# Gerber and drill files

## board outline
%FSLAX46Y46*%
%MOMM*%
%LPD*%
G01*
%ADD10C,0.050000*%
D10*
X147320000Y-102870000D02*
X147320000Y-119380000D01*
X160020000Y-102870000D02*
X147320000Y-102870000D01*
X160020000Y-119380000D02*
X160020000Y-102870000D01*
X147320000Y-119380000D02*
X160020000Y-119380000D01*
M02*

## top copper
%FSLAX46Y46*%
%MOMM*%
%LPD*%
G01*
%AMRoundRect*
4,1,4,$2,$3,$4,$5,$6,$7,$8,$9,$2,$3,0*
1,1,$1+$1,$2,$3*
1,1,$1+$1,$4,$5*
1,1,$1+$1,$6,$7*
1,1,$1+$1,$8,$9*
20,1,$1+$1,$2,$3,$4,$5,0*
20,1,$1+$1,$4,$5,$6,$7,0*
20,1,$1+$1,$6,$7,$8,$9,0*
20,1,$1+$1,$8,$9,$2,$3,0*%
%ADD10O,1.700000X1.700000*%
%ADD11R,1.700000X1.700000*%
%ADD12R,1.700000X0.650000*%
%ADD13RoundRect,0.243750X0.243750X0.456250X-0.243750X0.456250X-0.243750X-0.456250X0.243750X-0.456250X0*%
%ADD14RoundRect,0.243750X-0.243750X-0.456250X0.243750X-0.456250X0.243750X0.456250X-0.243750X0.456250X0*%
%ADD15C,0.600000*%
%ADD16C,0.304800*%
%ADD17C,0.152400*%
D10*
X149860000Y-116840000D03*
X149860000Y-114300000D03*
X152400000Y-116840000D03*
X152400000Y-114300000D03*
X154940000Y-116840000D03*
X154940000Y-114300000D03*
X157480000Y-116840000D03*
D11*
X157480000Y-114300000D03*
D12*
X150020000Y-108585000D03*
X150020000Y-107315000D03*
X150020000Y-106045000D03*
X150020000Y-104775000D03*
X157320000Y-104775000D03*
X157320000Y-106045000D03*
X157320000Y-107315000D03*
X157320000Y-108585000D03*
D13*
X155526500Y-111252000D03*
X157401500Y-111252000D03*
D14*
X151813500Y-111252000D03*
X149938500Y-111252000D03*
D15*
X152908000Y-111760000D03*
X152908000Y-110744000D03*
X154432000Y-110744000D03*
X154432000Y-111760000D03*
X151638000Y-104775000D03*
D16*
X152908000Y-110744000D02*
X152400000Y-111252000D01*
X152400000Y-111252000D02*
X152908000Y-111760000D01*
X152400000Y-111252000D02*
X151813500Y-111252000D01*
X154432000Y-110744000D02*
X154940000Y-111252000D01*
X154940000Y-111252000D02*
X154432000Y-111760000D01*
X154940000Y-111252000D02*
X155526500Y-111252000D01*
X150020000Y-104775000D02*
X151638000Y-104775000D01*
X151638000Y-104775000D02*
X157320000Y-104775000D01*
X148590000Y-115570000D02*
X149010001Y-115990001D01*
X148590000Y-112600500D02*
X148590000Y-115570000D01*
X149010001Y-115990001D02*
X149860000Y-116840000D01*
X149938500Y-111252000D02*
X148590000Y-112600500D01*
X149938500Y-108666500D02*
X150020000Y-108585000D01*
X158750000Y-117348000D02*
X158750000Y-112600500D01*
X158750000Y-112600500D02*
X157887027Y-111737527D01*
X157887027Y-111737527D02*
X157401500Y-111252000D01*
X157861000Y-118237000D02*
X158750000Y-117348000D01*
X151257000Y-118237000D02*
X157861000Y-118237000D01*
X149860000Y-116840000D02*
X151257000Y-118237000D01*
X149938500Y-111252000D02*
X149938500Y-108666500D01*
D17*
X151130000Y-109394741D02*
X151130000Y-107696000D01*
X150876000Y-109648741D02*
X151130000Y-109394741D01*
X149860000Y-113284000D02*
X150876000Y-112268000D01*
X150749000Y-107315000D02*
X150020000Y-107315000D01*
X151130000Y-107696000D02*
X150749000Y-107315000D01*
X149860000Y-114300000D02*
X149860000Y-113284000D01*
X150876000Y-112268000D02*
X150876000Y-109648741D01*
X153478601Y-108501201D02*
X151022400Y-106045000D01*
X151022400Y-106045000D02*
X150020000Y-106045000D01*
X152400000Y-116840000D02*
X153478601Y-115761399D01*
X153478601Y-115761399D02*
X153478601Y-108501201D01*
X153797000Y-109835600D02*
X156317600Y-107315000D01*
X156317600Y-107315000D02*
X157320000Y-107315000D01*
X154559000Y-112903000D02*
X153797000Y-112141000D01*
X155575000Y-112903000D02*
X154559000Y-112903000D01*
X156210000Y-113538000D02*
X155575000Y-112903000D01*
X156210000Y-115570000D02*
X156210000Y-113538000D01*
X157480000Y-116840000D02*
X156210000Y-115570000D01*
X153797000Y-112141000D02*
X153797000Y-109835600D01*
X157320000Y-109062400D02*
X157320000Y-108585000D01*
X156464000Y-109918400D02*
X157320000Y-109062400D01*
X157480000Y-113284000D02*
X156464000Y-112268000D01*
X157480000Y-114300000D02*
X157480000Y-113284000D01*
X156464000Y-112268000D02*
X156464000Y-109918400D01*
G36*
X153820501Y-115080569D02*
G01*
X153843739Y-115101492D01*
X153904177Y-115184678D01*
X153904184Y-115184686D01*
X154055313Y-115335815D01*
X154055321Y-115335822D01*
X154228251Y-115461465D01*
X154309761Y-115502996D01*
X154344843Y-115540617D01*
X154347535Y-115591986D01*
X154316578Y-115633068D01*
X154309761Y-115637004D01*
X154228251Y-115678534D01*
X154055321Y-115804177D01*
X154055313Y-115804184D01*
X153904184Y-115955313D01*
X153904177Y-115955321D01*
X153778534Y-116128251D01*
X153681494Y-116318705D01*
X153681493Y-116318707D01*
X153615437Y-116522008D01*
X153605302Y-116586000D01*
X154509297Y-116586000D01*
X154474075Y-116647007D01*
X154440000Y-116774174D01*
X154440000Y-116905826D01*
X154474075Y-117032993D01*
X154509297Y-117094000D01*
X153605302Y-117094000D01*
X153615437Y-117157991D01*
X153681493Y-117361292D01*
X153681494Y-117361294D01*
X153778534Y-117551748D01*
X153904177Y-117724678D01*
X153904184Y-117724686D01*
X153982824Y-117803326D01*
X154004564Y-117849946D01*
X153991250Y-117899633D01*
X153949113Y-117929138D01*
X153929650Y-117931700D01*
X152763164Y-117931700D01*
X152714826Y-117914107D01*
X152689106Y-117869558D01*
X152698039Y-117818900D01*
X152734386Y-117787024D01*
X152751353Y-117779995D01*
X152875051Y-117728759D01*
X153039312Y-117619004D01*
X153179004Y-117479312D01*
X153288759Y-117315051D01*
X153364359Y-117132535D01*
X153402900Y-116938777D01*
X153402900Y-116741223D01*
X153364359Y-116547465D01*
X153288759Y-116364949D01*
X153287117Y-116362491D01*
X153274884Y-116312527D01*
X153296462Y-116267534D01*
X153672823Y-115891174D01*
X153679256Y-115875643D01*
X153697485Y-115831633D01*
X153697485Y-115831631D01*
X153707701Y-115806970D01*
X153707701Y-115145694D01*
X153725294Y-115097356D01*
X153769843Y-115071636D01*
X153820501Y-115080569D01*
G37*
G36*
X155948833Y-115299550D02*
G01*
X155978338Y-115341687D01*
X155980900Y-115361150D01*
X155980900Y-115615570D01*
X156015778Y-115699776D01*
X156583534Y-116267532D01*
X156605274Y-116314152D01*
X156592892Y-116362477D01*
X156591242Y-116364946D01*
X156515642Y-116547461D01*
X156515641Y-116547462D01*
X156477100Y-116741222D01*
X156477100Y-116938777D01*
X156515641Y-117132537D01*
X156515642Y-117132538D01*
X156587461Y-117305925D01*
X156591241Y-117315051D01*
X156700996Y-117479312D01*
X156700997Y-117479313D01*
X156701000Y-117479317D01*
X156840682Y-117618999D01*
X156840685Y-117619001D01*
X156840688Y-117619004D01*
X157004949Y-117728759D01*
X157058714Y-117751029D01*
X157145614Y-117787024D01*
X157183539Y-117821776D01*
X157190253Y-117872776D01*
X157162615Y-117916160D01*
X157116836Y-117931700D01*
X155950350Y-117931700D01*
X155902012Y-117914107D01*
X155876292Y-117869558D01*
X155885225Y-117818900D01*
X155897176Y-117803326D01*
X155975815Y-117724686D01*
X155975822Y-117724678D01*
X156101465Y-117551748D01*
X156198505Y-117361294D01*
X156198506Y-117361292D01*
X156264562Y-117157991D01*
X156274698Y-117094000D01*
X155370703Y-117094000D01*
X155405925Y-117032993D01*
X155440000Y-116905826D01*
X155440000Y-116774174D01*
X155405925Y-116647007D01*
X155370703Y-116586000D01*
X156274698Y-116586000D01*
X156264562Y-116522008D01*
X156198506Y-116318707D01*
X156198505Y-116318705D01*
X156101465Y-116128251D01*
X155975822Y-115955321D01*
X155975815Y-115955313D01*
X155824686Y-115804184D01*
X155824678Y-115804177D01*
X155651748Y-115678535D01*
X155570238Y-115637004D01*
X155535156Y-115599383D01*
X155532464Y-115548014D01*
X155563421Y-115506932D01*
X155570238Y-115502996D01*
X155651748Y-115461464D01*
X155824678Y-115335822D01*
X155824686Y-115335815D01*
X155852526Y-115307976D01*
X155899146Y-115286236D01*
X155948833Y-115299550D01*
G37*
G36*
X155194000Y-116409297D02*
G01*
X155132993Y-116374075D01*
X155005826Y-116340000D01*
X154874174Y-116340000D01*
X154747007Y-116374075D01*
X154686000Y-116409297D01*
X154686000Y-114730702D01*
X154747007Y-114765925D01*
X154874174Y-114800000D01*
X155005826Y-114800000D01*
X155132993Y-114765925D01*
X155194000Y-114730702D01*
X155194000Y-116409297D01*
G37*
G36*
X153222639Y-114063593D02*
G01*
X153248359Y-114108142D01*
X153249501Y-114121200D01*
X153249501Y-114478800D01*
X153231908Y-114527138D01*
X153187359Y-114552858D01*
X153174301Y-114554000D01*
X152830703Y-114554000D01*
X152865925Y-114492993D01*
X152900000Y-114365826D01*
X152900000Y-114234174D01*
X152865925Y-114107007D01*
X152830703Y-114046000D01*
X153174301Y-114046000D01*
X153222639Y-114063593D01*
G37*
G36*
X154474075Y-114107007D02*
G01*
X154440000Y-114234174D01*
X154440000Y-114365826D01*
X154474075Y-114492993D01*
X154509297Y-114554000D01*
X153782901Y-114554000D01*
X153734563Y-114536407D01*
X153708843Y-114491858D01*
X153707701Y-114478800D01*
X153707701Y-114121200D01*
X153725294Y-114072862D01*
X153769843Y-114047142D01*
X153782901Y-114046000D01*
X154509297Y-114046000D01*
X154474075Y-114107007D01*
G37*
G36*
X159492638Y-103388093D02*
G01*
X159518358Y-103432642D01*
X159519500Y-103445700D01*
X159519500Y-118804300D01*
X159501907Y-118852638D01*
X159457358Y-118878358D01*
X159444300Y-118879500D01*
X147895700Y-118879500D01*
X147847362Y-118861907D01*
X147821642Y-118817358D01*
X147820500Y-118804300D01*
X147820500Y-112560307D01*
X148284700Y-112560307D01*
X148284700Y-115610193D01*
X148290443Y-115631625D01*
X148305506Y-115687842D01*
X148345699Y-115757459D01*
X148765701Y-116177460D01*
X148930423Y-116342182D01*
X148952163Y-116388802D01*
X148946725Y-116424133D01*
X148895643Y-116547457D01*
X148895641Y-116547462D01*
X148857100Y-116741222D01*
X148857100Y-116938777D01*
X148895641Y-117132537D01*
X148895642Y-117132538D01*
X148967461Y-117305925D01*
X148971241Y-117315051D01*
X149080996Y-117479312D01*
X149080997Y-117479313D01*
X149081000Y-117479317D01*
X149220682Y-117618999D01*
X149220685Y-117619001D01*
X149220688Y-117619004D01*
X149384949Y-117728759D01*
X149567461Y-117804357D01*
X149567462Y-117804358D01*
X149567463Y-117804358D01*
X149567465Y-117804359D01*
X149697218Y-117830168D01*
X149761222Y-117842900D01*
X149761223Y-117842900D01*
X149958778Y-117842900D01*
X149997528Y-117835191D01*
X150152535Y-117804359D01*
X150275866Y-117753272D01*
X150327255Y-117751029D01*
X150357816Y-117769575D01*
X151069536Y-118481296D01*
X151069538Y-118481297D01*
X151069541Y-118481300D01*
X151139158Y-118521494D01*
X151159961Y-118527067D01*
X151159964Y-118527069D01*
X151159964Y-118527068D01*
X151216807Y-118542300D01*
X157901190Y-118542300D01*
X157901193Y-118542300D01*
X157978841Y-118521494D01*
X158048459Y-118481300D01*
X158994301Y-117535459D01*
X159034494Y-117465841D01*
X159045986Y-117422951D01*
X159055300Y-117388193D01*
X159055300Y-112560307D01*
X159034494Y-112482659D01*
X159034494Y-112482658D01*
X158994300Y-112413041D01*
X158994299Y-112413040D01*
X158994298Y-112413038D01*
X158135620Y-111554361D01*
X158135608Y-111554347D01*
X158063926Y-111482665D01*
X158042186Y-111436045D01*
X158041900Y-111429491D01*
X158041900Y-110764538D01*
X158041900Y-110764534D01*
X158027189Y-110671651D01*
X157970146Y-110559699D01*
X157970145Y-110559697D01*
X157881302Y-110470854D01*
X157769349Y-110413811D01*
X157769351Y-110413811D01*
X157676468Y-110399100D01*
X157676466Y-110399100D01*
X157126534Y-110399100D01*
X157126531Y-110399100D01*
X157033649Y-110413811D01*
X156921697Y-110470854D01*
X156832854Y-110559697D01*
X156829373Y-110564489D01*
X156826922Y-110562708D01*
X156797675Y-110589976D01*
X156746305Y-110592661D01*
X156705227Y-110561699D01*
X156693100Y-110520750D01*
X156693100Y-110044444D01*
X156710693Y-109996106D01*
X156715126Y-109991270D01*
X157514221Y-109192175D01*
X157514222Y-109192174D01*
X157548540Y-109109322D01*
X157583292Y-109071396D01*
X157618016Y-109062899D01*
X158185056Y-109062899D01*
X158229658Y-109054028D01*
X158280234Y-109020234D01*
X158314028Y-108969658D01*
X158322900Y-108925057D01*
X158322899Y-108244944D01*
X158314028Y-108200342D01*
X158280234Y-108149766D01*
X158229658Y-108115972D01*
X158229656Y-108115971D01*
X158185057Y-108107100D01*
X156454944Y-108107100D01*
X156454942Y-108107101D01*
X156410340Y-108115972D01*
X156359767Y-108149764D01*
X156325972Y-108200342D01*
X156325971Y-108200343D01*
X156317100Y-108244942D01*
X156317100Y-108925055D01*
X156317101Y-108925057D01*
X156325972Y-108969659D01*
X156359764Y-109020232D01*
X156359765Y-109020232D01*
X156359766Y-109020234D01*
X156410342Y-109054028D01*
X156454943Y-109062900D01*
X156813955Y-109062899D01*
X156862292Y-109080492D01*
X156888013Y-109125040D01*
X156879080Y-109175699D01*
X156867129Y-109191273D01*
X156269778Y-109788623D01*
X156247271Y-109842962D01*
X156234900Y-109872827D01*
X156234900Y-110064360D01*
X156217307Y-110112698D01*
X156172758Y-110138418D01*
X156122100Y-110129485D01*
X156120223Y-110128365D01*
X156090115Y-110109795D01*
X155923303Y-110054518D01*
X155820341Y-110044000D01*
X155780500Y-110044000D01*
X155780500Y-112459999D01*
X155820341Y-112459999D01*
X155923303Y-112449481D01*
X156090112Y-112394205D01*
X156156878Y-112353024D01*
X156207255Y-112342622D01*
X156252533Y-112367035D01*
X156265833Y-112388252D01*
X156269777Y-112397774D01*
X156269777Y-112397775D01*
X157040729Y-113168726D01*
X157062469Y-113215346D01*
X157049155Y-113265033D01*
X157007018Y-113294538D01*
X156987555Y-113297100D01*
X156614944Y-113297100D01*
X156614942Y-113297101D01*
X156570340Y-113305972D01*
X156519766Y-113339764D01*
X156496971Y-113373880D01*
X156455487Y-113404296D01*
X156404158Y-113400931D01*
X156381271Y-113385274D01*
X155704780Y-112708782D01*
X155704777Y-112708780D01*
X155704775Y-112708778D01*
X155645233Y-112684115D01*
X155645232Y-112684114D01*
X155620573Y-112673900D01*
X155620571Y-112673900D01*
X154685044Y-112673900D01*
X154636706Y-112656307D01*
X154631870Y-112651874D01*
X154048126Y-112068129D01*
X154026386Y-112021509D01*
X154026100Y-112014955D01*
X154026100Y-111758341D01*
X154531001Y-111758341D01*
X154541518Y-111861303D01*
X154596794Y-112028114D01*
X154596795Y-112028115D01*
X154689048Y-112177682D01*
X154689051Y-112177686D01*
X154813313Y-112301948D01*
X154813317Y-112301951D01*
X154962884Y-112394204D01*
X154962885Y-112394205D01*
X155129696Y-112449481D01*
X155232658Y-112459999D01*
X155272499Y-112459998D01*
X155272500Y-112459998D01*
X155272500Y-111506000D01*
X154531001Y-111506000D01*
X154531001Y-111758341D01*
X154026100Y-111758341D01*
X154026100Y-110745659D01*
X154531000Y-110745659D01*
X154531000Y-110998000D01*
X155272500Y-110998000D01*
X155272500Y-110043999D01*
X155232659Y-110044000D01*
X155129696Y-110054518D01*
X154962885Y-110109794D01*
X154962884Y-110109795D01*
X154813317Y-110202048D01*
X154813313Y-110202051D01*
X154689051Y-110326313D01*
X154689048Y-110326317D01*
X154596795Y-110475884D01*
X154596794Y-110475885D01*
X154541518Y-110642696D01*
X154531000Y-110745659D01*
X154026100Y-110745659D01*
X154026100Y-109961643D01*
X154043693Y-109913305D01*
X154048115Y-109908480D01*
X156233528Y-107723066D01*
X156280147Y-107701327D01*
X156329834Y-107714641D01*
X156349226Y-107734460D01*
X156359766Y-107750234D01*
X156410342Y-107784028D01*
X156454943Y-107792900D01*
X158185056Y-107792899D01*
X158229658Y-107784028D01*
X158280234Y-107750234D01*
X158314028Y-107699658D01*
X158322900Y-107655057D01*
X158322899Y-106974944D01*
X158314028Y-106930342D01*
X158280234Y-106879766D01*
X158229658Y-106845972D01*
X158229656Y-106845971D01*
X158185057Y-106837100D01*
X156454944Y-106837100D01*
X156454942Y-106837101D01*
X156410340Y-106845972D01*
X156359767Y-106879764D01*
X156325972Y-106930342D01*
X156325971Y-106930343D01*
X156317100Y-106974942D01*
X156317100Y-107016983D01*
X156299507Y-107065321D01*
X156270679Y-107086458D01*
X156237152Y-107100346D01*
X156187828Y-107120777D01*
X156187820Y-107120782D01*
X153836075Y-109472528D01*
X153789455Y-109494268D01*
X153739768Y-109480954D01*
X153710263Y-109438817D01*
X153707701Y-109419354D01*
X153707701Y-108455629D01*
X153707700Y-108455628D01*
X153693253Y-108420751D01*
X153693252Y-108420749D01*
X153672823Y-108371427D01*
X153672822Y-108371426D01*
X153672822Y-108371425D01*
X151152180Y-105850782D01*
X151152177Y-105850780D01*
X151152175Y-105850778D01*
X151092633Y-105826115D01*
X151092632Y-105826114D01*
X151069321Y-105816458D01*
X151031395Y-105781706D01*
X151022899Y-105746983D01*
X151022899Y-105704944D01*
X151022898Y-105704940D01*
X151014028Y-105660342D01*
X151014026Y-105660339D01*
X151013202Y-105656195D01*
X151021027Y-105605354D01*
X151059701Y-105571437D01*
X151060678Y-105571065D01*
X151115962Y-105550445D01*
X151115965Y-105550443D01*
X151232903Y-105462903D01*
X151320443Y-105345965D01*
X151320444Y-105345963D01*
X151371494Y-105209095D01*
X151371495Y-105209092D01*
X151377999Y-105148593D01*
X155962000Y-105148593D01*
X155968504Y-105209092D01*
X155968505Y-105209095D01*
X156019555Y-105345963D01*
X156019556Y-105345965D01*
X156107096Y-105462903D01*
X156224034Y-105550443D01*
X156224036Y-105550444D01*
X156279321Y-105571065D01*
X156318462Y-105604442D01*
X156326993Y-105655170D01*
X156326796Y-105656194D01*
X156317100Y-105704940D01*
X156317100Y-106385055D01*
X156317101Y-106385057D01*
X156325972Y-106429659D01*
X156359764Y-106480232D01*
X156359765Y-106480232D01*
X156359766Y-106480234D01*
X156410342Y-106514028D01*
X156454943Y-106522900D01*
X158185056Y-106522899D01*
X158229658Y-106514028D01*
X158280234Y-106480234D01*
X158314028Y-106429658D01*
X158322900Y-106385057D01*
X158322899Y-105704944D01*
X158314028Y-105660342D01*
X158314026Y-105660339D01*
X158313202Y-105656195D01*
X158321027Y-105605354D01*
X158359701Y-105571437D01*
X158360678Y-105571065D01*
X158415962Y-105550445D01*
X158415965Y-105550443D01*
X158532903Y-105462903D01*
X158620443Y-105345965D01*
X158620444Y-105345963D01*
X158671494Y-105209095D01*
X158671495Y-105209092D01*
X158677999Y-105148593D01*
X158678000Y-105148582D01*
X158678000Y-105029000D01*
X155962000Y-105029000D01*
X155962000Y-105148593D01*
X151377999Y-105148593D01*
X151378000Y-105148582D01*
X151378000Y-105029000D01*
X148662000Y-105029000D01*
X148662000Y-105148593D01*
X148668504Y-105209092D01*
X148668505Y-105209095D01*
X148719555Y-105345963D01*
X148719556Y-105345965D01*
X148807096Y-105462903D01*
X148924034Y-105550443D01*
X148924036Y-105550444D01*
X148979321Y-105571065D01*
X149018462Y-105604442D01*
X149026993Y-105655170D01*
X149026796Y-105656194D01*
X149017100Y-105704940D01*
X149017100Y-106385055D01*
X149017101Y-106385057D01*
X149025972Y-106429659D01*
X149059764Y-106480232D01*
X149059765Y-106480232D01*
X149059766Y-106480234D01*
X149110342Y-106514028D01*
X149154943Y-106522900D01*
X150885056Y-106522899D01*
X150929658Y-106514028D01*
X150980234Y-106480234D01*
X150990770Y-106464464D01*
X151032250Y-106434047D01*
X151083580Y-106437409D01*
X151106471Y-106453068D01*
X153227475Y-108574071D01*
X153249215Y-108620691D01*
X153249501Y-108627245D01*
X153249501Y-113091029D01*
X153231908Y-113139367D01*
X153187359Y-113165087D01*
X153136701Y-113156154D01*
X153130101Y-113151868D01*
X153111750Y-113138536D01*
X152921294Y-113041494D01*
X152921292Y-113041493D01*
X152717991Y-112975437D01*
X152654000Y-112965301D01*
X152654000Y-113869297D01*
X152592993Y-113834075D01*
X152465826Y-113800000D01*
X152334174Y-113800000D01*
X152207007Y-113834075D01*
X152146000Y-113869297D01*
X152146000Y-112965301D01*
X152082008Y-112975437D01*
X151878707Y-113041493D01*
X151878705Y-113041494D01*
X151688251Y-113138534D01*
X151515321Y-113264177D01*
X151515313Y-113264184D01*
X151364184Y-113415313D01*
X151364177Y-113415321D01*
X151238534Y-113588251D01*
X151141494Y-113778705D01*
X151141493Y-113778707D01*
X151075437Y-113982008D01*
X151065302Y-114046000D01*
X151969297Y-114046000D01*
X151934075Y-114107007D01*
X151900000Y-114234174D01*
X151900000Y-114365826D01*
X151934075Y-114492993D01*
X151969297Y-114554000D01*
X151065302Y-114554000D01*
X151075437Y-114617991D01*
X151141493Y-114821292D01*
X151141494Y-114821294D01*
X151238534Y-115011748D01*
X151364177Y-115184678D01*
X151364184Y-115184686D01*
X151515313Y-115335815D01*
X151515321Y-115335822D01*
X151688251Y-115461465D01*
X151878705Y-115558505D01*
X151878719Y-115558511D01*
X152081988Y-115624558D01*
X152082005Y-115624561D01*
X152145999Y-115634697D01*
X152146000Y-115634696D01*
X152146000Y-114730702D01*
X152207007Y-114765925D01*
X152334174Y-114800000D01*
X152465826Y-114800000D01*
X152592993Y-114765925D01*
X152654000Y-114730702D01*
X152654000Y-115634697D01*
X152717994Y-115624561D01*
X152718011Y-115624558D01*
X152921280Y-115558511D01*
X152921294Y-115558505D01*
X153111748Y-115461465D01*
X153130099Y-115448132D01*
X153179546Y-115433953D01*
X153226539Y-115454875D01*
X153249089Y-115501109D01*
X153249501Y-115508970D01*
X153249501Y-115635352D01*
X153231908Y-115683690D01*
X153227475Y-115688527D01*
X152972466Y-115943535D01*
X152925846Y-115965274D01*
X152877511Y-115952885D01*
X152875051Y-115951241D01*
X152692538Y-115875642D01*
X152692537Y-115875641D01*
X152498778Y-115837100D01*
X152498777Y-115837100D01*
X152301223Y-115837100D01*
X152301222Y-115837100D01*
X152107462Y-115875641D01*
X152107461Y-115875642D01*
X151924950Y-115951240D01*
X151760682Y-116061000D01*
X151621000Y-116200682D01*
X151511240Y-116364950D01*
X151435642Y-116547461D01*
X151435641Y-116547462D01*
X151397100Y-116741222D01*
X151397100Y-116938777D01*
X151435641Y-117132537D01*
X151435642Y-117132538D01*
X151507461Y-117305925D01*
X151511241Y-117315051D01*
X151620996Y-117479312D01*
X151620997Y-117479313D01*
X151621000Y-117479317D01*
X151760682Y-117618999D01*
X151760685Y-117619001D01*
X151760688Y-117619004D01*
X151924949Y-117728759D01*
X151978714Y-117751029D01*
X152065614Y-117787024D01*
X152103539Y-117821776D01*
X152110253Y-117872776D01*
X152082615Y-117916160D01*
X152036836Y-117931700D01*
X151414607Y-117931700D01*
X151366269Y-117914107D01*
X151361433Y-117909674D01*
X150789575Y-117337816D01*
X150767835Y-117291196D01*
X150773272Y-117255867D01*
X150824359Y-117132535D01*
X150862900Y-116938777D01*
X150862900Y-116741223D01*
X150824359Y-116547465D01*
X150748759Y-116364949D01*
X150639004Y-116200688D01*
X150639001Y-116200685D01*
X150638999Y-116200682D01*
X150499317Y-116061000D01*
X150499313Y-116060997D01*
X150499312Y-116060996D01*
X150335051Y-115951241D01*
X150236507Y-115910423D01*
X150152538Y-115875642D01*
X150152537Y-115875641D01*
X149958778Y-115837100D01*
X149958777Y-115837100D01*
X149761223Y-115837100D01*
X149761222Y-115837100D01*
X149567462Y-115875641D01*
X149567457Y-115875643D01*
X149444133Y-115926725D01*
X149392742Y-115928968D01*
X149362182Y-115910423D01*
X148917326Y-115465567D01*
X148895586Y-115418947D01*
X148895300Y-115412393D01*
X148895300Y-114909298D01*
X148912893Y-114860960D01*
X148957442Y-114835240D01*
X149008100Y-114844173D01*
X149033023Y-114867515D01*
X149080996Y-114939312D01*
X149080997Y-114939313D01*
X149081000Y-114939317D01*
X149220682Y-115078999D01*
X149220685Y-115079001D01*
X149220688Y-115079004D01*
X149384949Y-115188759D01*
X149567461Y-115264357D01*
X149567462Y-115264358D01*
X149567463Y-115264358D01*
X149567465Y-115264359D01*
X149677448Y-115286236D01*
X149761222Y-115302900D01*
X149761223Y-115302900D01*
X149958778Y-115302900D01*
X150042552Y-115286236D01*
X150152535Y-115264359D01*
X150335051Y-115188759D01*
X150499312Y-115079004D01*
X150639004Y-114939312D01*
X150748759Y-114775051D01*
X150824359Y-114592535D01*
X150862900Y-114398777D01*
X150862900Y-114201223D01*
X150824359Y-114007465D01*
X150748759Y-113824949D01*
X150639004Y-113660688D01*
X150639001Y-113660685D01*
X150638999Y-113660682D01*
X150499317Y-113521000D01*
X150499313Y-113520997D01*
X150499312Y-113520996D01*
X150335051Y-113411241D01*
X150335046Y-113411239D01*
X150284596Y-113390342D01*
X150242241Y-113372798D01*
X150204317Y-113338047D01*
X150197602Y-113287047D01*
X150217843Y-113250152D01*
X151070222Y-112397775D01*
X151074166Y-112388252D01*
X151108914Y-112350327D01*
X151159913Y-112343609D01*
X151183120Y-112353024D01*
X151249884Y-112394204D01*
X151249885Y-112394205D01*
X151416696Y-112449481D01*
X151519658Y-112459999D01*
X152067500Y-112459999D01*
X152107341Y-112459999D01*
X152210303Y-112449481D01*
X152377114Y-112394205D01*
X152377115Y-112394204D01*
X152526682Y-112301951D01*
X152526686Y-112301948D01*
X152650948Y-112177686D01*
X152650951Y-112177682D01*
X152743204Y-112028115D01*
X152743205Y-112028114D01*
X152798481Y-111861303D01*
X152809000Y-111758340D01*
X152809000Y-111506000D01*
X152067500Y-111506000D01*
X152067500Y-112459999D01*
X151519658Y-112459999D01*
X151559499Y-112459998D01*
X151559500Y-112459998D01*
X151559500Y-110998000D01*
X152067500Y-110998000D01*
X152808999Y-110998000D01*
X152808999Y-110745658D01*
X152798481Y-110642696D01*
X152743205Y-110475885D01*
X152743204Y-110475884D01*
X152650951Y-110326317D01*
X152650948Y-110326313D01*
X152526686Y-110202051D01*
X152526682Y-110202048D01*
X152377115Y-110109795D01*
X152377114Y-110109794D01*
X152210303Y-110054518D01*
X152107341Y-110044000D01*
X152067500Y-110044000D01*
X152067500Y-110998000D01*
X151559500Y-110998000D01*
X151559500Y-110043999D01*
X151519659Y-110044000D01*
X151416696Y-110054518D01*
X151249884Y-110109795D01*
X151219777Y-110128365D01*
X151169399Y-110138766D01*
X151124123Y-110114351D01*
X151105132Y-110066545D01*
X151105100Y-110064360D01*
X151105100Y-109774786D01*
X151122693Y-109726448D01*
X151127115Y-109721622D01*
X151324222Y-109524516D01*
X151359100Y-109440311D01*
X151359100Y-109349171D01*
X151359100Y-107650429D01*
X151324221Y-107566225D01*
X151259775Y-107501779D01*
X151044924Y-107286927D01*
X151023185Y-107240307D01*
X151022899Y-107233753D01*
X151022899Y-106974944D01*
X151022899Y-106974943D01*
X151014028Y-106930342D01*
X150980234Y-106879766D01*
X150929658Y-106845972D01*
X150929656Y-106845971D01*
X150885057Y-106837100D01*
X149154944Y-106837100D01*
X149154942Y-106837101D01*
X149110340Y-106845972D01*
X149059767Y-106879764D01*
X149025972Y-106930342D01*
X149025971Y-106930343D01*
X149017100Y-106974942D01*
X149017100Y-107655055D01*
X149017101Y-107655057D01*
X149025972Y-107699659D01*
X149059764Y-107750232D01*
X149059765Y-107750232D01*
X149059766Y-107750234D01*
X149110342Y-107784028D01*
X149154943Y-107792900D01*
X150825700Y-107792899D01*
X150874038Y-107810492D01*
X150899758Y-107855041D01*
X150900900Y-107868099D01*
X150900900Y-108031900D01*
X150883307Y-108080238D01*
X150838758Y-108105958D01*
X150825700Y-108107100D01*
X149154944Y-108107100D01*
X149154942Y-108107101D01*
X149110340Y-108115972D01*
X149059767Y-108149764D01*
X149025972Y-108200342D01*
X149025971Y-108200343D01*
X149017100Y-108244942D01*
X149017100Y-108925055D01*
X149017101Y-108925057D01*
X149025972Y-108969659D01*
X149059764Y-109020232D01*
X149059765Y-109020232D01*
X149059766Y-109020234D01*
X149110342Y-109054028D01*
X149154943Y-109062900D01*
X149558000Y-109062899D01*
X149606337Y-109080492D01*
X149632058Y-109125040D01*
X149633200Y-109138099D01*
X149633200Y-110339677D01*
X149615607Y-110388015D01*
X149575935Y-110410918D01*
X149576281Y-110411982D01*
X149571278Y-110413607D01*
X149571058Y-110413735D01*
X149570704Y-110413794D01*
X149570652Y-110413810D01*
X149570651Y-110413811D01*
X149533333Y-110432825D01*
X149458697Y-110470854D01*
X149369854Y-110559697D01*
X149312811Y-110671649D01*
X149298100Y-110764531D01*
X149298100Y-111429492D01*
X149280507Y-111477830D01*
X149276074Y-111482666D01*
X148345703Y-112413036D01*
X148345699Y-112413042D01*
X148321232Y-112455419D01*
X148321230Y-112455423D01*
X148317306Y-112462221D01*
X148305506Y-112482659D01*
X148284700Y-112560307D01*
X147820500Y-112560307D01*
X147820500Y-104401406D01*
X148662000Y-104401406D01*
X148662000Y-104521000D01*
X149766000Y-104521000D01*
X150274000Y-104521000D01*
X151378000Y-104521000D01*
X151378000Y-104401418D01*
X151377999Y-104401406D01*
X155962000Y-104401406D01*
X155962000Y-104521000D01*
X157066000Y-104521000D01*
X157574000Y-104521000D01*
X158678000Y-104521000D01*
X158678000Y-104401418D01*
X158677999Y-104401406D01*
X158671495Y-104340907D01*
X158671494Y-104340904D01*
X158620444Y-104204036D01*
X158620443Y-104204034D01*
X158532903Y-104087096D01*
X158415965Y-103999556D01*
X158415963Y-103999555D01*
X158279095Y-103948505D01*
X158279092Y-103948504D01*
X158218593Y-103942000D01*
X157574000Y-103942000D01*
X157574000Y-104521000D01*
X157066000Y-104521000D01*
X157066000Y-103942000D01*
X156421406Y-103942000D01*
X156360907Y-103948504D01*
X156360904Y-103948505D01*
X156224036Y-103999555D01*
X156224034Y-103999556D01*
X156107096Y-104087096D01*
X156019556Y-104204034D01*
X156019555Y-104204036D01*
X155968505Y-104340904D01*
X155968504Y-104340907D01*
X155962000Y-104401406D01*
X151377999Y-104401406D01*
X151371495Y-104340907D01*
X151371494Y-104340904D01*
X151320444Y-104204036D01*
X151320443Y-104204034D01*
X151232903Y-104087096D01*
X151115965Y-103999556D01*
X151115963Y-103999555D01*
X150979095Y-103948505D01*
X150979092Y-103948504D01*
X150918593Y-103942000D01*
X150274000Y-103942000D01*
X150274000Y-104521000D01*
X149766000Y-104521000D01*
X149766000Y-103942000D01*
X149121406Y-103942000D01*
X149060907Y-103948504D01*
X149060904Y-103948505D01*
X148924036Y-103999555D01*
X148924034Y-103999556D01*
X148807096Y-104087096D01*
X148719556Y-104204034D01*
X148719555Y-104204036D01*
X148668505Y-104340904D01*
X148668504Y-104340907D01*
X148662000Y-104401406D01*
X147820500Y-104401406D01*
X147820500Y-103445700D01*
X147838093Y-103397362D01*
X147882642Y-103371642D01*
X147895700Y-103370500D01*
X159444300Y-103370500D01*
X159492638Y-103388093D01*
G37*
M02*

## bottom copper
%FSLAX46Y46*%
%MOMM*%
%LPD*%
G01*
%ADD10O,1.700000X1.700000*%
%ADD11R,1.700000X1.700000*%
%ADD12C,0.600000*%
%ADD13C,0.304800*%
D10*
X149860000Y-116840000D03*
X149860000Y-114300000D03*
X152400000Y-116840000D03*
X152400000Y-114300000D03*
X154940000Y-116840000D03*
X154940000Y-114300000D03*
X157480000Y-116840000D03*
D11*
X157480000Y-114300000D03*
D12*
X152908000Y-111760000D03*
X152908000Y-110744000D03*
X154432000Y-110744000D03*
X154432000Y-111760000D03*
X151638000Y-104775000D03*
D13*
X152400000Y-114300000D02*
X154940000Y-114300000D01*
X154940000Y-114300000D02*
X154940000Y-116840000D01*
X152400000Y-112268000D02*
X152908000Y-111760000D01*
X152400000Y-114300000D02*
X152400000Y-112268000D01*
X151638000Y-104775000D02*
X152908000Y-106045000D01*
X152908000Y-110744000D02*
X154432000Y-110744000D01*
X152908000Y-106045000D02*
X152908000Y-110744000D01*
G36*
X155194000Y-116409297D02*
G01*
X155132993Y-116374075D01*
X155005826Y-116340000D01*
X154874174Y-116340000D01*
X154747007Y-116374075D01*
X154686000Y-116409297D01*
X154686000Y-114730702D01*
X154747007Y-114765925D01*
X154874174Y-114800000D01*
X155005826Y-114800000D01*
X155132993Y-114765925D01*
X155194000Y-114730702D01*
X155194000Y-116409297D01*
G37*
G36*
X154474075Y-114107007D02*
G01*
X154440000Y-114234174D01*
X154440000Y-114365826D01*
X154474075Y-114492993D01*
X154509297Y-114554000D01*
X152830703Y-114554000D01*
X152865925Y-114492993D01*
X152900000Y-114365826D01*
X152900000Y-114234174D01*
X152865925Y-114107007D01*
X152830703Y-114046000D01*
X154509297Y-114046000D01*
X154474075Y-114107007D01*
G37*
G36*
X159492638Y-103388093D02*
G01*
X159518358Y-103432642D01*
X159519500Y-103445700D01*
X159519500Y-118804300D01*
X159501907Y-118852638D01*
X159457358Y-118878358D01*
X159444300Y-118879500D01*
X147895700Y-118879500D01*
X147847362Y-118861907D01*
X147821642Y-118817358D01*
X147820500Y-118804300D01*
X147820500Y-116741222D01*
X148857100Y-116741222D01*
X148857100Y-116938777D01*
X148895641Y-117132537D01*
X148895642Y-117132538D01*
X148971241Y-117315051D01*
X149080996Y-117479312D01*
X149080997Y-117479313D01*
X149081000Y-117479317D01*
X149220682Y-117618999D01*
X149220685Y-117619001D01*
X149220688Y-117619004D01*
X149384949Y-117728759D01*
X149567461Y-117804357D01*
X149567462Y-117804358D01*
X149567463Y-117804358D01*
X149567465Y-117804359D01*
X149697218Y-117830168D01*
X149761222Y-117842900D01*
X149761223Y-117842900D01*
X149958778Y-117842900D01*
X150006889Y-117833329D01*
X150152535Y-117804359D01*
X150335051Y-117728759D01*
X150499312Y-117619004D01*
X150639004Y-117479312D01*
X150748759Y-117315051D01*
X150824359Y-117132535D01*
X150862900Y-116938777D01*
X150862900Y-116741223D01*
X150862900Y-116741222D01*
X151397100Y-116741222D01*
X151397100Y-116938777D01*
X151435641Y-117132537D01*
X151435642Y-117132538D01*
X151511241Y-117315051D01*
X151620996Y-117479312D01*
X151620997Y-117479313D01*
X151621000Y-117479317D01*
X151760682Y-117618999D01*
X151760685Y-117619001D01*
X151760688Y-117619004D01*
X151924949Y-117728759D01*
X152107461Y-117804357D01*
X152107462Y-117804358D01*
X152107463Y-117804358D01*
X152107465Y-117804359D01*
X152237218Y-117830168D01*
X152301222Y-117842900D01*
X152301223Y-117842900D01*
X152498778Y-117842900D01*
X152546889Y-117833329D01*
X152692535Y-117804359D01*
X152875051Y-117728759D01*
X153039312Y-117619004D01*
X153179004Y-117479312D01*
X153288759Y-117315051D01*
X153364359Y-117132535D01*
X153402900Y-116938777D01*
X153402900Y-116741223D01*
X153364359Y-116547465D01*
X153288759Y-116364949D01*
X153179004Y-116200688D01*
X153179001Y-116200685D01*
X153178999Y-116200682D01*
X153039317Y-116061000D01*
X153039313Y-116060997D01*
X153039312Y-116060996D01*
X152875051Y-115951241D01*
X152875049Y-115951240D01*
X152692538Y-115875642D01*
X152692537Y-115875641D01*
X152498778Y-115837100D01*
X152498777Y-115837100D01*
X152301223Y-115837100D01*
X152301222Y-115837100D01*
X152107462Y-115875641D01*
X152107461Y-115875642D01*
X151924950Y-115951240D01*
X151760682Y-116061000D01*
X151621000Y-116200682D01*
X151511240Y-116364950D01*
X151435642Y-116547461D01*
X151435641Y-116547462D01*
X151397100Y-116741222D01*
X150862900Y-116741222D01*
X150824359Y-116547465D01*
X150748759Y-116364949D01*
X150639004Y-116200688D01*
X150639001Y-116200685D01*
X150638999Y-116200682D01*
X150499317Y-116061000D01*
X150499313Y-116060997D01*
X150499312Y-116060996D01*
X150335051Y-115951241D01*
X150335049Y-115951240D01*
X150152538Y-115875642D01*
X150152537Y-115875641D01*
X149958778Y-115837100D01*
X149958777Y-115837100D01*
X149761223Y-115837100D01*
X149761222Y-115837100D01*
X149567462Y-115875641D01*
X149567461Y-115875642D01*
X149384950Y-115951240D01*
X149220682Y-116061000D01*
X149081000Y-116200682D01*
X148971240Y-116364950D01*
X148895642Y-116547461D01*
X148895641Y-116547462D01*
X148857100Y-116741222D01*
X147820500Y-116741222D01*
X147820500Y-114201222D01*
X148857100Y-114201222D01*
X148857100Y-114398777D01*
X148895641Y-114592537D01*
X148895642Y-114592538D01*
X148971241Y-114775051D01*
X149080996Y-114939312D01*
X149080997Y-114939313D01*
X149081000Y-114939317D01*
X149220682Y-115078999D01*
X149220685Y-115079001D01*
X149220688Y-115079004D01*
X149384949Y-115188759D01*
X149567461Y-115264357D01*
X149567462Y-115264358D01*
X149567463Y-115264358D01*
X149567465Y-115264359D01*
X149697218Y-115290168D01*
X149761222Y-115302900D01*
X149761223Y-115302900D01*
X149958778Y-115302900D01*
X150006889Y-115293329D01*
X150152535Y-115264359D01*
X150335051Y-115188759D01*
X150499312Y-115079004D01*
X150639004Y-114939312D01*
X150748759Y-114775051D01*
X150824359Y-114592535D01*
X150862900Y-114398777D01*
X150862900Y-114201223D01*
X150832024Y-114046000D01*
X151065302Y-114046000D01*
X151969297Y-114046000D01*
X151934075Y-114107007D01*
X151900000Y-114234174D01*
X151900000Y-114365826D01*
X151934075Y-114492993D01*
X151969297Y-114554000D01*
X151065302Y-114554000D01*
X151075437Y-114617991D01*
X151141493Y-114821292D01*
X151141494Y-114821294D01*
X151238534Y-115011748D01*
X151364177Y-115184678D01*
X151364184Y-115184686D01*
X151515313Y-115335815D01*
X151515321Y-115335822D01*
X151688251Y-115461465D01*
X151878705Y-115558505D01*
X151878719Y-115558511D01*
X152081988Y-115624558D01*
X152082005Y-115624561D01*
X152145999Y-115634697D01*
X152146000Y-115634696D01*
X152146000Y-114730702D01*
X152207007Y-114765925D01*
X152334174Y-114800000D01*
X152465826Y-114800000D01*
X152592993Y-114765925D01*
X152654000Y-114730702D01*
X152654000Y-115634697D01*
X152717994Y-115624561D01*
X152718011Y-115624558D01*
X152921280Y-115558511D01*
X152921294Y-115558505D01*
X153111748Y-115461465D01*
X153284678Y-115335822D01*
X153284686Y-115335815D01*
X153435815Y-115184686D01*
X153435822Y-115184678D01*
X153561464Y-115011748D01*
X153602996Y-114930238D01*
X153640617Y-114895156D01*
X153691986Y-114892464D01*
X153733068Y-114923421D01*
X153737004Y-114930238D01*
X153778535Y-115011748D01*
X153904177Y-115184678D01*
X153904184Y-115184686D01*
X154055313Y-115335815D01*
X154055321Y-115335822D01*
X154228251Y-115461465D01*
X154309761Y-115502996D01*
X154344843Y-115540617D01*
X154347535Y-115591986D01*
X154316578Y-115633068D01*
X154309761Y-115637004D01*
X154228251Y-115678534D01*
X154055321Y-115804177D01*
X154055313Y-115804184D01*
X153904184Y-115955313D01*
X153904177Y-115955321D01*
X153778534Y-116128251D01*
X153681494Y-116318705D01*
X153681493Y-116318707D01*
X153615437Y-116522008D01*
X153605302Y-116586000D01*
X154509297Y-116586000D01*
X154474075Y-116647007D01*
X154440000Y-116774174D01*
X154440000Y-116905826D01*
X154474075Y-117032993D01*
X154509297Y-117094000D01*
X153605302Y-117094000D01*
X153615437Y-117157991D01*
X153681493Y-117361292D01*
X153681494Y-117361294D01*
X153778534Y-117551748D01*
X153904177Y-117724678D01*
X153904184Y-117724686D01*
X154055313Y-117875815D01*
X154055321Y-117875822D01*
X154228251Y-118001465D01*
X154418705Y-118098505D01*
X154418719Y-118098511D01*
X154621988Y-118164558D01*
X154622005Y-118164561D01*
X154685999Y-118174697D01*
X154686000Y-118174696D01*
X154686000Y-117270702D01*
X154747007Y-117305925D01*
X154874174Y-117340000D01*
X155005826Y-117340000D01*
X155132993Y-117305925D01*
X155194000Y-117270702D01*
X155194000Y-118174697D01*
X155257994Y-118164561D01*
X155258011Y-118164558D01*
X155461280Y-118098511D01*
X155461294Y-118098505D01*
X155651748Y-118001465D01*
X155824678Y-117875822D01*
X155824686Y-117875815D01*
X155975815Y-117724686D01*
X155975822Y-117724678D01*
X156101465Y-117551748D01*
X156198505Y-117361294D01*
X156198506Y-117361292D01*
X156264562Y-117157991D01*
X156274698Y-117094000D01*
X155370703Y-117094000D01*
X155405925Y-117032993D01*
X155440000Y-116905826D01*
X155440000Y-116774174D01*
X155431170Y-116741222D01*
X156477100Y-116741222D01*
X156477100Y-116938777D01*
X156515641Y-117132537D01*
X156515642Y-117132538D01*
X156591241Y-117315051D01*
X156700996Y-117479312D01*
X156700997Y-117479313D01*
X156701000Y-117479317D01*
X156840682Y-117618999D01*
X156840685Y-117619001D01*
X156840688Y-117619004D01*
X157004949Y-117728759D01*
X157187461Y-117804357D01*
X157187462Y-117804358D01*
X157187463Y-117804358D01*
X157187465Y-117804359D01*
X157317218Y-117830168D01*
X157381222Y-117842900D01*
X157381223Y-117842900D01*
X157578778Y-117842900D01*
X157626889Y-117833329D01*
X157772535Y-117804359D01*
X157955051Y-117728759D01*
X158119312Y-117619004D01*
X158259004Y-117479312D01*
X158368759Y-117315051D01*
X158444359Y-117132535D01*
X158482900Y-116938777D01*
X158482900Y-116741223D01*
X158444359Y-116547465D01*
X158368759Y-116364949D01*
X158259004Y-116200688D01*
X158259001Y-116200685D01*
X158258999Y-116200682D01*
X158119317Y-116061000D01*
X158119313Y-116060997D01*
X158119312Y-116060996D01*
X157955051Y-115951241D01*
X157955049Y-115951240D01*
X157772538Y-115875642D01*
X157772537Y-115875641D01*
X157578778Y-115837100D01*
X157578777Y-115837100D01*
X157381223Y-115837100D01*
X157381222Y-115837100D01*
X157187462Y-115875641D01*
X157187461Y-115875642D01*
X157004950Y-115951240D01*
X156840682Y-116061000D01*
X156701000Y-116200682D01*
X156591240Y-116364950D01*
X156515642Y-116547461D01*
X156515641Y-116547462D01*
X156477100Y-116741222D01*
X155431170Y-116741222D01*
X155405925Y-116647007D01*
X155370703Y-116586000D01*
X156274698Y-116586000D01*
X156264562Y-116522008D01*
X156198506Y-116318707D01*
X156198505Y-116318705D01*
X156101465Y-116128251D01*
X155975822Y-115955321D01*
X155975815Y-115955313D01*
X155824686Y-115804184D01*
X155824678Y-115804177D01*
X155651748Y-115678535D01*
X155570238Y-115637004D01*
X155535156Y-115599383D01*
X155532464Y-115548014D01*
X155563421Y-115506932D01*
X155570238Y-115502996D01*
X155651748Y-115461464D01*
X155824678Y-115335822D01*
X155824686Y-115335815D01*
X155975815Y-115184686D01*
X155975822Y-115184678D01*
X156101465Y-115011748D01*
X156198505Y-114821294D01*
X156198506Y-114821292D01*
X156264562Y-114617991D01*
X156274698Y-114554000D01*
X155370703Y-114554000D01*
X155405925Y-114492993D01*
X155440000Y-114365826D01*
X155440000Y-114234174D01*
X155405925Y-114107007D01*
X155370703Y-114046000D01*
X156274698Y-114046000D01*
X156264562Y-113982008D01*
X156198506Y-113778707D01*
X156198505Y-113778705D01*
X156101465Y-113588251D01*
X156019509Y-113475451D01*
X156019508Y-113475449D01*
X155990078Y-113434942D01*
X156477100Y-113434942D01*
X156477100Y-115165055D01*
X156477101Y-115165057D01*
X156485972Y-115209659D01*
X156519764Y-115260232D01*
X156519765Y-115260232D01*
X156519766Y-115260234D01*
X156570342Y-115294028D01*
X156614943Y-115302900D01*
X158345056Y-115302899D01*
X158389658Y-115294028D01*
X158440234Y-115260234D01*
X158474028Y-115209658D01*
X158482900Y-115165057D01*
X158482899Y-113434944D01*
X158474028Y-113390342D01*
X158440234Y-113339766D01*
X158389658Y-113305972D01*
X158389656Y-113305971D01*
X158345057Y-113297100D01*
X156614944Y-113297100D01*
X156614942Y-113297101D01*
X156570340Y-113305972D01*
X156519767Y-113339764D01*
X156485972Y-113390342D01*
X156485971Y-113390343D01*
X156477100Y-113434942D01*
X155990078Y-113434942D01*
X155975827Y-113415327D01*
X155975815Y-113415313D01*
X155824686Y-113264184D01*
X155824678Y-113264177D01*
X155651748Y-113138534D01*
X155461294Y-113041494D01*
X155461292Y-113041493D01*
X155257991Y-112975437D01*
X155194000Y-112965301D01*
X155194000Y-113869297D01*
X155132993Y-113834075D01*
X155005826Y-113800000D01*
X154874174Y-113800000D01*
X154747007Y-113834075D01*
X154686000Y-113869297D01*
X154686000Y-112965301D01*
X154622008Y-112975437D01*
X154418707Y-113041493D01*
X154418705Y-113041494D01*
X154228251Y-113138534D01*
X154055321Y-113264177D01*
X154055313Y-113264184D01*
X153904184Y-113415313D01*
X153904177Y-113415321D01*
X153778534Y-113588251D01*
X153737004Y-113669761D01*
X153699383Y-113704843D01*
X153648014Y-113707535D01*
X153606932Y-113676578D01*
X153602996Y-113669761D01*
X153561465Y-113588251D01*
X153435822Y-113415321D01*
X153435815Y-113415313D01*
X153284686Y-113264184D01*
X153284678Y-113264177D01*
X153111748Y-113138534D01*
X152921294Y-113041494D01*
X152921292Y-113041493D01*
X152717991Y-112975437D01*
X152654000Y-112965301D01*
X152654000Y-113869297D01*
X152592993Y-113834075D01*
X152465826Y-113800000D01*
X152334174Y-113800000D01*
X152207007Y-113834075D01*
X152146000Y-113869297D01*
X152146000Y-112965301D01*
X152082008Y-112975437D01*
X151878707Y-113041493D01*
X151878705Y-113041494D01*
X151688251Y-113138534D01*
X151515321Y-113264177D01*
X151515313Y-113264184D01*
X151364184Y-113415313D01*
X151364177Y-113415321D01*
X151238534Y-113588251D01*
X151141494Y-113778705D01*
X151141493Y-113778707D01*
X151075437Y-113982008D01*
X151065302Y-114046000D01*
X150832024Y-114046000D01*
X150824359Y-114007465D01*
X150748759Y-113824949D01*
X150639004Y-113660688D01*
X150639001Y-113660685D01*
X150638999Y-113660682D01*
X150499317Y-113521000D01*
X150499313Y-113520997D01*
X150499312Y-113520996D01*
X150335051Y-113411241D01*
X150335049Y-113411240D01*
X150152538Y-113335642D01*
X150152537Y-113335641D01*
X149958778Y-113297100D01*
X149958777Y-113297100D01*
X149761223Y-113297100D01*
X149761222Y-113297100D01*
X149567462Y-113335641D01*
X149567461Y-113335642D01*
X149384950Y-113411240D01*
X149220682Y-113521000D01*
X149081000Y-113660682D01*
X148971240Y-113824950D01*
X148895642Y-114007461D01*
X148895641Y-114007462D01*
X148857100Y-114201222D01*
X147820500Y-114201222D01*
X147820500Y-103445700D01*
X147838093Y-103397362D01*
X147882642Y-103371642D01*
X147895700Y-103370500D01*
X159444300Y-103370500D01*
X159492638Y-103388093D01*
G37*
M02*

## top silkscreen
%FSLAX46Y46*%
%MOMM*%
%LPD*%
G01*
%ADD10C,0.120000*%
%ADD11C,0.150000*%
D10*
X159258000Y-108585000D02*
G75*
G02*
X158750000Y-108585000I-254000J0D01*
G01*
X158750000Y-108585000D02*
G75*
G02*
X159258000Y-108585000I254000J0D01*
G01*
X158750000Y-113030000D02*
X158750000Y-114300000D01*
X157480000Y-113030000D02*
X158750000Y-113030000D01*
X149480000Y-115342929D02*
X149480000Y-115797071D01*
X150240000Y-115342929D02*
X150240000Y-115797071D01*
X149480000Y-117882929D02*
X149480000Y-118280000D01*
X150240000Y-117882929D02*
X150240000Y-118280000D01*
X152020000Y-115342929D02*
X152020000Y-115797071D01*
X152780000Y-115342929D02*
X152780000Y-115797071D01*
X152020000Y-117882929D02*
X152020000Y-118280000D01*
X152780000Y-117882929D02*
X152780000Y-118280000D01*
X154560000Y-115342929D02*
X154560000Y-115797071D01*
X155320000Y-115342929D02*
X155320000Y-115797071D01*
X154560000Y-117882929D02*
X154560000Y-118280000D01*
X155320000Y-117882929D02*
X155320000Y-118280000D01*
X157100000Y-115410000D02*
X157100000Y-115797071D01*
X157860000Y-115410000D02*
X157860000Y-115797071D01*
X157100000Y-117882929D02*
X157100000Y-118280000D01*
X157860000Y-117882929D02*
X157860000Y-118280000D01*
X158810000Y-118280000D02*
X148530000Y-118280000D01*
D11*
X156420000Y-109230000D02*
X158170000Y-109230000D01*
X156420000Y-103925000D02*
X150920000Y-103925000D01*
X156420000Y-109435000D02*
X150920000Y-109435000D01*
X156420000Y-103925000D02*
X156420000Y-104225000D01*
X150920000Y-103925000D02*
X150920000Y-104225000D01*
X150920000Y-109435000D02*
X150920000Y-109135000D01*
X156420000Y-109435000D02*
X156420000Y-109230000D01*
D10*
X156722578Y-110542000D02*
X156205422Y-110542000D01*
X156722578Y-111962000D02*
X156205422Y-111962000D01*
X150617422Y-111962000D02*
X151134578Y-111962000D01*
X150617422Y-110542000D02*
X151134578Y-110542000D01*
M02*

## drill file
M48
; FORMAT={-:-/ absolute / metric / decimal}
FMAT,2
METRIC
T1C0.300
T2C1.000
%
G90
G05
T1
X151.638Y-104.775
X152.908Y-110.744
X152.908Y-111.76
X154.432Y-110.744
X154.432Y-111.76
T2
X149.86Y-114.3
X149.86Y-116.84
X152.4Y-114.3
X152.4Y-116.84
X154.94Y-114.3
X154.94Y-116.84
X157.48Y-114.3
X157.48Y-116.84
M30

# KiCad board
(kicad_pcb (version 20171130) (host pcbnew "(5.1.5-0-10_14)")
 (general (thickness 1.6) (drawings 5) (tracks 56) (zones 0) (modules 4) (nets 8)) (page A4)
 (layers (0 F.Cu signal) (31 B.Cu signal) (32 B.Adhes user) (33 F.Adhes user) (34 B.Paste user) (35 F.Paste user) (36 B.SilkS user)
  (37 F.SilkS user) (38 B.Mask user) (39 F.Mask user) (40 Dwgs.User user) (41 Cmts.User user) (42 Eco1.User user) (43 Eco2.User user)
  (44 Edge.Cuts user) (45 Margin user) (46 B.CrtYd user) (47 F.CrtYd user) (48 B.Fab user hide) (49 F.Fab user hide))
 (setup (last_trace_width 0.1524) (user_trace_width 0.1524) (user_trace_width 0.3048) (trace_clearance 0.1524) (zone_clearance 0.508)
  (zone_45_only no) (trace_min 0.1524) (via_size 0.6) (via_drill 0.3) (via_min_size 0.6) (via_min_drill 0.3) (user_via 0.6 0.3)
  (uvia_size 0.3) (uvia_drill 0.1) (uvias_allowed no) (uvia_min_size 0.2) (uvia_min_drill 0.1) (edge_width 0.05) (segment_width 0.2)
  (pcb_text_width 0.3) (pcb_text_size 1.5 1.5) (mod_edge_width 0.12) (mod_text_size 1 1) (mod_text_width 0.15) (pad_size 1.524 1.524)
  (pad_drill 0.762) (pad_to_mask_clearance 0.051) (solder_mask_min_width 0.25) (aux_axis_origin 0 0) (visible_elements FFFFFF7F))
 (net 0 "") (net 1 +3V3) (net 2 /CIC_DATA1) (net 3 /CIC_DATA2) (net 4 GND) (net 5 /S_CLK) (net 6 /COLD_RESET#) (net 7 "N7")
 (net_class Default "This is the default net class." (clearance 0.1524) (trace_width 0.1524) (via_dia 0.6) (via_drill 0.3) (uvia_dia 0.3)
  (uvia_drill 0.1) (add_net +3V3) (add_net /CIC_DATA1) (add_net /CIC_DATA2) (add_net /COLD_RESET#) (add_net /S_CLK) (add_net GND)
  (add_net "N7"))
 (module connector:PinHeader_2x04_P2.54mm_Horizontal (layer F.Cu) (at 157.48 114.3 270)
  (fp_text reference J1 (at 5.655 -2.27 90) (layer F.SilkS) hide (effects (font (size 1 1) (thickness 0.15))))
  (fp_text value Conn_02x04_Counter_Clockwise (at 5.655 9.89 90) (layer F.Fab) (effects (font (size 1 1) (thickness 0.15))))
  (fp_line (start -1.27 -1.27) (end 0 -1.27) (layer F.SilkS) (width 0.12))
  (fp_line (start -1.27 0) (end -1.27 -1.27) (layer F.SilkS) (width 0.12))
  (fp_line (start 1.042929 8) (end 1.497071 8) (layer F.SilkS) (width 0.12))
  (fp_line (start 1.042929 7.24) (end 1.497071 7.24) (layer F.SilkS) (width 0.12))
  (fp_line (start 3.582929 8) (end 3.98 8) (layer F.SilkS) (width 0.12))
  (fp_line (start 3.582929 7.24) (end 3.98 7.24) (layer F.SilkS) (width 0.12))
  (fp_line (start 1.042929 5.46) (end 1.497071 5.46) (layer F.SilkS) (width 0.12))
  (fp_line (start 1.042929 4.7) (end 1.497071 4.7) (layer F.SilkS) (width 0.12))
  (fp_line (start 3.582929 5.46) (end 3.98 5.46) (layer F.SilkS) (width 0.12))
  (fp_line (start 3.582929 4.7) (end 3.98 4.7) (layer F.SilkS) (width 0.12))
  (fp_line (start 1.042929 2.92) (end 1.497071 2.92) (layer F.SilkS) (width 0.12))
  (fp_line (start 1.042929 2.16) (end 1.497071 2.16) (layer F.SilkS) (width 0.12))
  (fp_line (start 3.582929 2.92) (end 3.98 2.92) (layer F.SilkS) (width 0.12))
  (fp_line (start 3.582929 2.16) (end 3.98 2.16) (layer F.SilkS) (width 0.12))
  (fp_line (start 1.11 0.38) (end 1.497071 0.38) (layer F.SilkS) (width 0.12))
  (fp_line (start 1.11 -0.38) (end 1.497071 -0.38) (layer F.SilkS) (width 0.12))
  (fp_line (start 3.582929 0.38) (end 3.98 0.38) (layer F.SilkS) (width 0.12))
  (fp_line (start 3.582929 -0.38) (end 3.98 -0.38) (layer F.SilkS) (width 0.12))
  (fp_line (start 3.98 -1.33) (end 3.98 8.95) (layer F.SilkS) (width 0.12))
  (pad 8 thru_hole oval (at 2.54 7.62 270) (size 1.7 1.7) (drill 1) (layers *.Cu *.Mask) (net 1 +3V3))
  (pad 7 thru_hole oval (at 0 7.62 270) (size 1.7 1.7) (drill 1) (layers *.Cu *.Mask) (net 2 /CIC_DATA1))
  (pad 6 thru_hole oval (at 2.54 5.08 270) (size 1.7 1.7) (drill 1) (layers *.Cu *.Mask) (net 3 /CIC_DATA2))
  (pad 5 thru_hole oval (at 0 5.08 270) (size 1.7 1.7) (drill 1) (layers *.Cu *.Mask) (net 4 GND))
  (pad 4 thru_hole oval (at 2.54 2.54 270) (size 1.7 1.7) (drill 1) (layers *.Cu *.Mask) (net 4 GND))
  (pad 3 thru_hole oval (at 0 2.54 270) (size 1.7 1.7) (drill 1) (layers *.Cu *.Mask) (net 4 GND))
  (pad 2 thru_hole oval (at 2.54 0 270) (size 1.7 1.7) (drill 1) (layers *.Cu *.Mask) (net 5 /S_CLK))
  (pad 1 thru_hole rect (at 0 0 270) (size 1.7 1.7) (drill 1) (layers *.Cu *.Mask) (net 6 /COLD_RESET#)))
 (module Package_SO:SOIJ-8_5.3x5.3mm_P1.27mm (layer F.Cu) (at 153.67 106.68 180)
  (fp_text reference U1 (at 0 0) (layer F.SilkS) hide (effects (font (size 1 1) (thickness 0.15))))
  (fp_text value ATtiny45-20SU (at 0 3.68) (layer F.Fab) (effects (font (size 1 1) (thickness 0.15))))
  (fp_line (start -2.75 -2.55) (end -4.5 -2.55) (layer F.SilkS) (width 0.15))
  (fp_line (start -2.75 2.755) (end 2.75 2.755) (layer F.SilkS) (width 0.15))
  (fp_line (start -2.75 -2.755) (end 2.75 -2.755) (layer F.SilkS) (width 0.15))
  (fp_line (start -2.75 2.755) (end -2.75 2.455) (layer F.SilkS) (width 0.15))
  (fp_line (start 2.75 2.755) (end 2.75 2.455) (layer F.SilkS) (width 0.15))
  (fp_line (start 2.75 -2.755) (end 2.75 -2.455) (layer F.SilkS) (width 0.15))
  (fp_line (start -2.75 -2.755) (end -2.75 -2.55) (layer F.SilkS) (width 0.15))
  (pad 8 smd rect (at 3.65 -1.905 180) (size 1.7 0.65) (layers F.Cu F.Paste F.Mask) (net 1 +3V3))
  (pad 7 smd rect (at 3.65 -0.635 180) (size 1.7 0.65) (layers F.Cu F.Paste F.Mask) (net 2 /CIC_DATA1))
  (pad 6 smd rect (at 3.65 0.635 180) (size 1.7 0.65) (layers F.Cu F.Paste F.Mask) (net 3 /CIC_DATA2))
  (pad 5 smd rect (at 3.65 1.905 180) (size 1.7 0.65) (layers F.Cu F.Paste F.Mask) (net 4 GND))
  (pad 4 smd rect (at -3.65 1.905 180) (size 1.7 0.65) (layers F.Cu F.Paste F.Mask) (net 4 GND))
  (pad 3 smd rect (at -3.65 0.635 180) (size 1.7 0.65) (layers F.Cu F.Paste F.Mask) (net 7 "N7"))
  (pad 2 smd rect (at -3.65 -0.635 180) (size 1.7 0.65) (layers F.Cu F.Paste F.Mask) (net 5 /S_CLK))
  (pad 1 smd rect (at -3.65 -1.905 180) (size 1.7 0.65) (layers F.Cu F.Paste F.Mask) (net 6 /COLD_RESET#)))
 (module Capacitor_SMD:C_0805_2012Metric (layer F.Cu) (at 156.464 111.252 180)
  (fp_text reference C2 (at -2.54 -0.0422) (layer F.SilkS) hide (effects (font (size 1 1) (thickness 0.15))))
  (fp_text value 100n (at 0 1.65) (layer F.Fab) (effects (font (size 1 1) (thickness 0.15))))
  (fp_line (start -0.258578 0.71) (end 0.258578 0.71) (layer F.SilkS) (width 0.12))
  (fp_line (start -0.258578 -0.71) (end 0.258578 -0.71) (layer F.SilkS) (width 0.12))
  (pad 2 smd roundrect (at 0.9375 0 180) (size 0.975 1.4) (layers F.Cu F.Paste F.Mask) (roundrect_rratio 0.25) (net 4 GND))
  (pad 1 smd roundrect (at -0.9375 0 180) (size 0.975 1.4) (layers F.Cu F.Paste F.Mask) (roundrect_rratio 0.25) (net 1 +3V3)))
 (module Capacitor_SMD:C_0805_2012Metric (layer F.Cu) (at 150.876 111.252)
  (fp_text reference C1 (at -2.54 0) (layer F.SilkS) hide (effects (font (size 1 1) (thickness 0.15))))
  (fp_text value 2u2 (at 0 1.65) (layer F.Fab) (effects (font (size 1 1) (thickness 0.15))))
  (fp_line (start -0.258578 0.71) (end 0.258578 0.71) (layer F.SilkS) (width 0.12))
  (fp_line (start -0.258578 -0.71) (end 0.258578 -0.71) (layer F.SilkS) (width 0.12))
  (pad 2 smd roundrect (at 0.9375 0) (size 0.975 1.4) (layers F.Cu F.Paste F.Mask) (roundrect_rratio 0.25) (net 4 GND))
  (pad 1 smd roundrect (at -0.9375 0) (size 0.975 1.4) (layers F.Cu F.Paste F.Mask) (roundrect_rratio 0.25) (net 1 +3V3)))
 (gr_circle (center 159.004 108.585) (end 159.004 108.839) (layer F.SilkS) (width 0.12))
 (gr_line (start 147.32 102.87) (end 147.32 119.38) (layer Edge.Cuts) (width 0.05))
 (gr_line (start 160.02 102.87) (end 147.32 102.87) (layer Edge.Cuts) (width 0.05))
 (gr_line (start 160.02 119.38) (end 160.02 102.87) (layer Edge.Cuts) (width 0.05))
 (gr_line (start 147.32 119.38) (end 160.02 119.38) (layer Edge.Cuts) (width 0.05))
 (via (at 152.908 111.76) (size 0.6) (drill 0.3) (layers F.Cu B.Cu) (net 4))
 (via (at 152.908 110.744) (size 0.6) (drill 0.3) (layers F.Cu B.Cu) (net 4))
 (via (at 154.432 110.744) (size 0.6) (drill 0.3) (layers F.Cu B.Cu) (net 4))
 (via (at 154.432 111.76) (size 0.6) (drill 0.3) (layers F.Cu B.Cu) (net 4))
 (segment (start 152.908 110.744) (end 152.4 111.252) (width 0.3048) (layer F.Cu) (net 4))
 (segment (start 152.4 111.252) (end 152.908 111.76) (width 0.3048) (layer F.Cu) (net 4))
 (segment (start 152.4 111.252) (end 151.8135 111.252) (width 0.3048) (layer F.Cu) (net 4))
 (segment (start 154.432 110.744) (end 154.94 111.252) (width 0.3048) (layer F.Cu) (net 4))
 (segment (start 154.94 111.252) (end 154.432 111.76) (width 0.3048) (layer F.Cu) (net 4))
 (segment (start 154.94 111.252) (end 155.5265 111.252) (width 0.3048) (layer F.Cu) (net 4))
 (segment (start 152.4 114.3) (end 154.94 114.3) (width 0.3048) (layer B.Cu) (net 4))
 (segment (start 154.94 114.3) (end 154.94 116.84) (width 0.3048) (layer B.Cu) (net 4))
 (segment (start 152.4 112.268) (end 152.908 111.76) (width 0.3048) (layer B.Cu) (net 4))
 (segment (start 152.4 114.3) (end 152.4 112.268) (width 0.3048) (layer B.Cu) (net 4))
 (via (at 151.638 104.775) (size 0.6) (drill 0.3) (layers F.Cu B.Cu) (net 4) (status 1000000))
 (segment (start 150.02 104.775) (end 151.638 104.775) (width 0.3048) (layer F.Cu) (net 4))
 (segment (start 151.638 104.775) (end 152.908 106.045) (width 0.3048) (layer B.Cu) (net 4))
 (segment (start 151.638 104.775) (end 157.32 104.775) (width 0.3048) (layer F.Cu) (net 4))
 (segment (start 152.908 110.744) (end 154.432 110.744) (width 0.3048) (layer B.Cu) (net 4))
 (segment (start 152.908 106.045) (end 152.908 110.744) (width 0.3048) (layer B.Cu) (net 4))
 (segment (start 148.59 115.57) (end 149.010001 115.990001) (width 0.3048) (layer F.Cu) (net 1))
 (segment (start 148.59 112.6005) (end 148.59 115.57) (width 0.3048) (layer F.Cu) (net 1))
 (segment (start 149.010001 115.990001) (end 149.86 116.84) (width 0.3048) (layer F.Cu) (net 1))
 (segment (start 149.9385 111.252) (end 148.59 112.6005) (width 0.3048) (layer F.Cu) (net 1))
 (segment (start 149.9385 108.6665) (end 150.02 108.585) (width 0.3048) (layer F.Cu) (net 1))
 (segment (start 158.75 117.348) (end 158.75 112.6005) (width 0.3048) (layer F.Cu) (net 1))
 (segment (start 158.75 112.6005) (end 157.887027 111.737527) (width 0.3048) (layer F.Cu) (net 1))
 (segment (start 157.887027 111.737527) (end 157.4015 111.252) (width 0.3048) (layer F.Cu) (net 1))
 (segment (start 157.861 118.237) (end 158.75 117.348) (width 0.3048) (layer F.Cu) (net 1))
 (segment (start 151.257 118.237) (end 157.861 118.237) (width 0.3048) (layer F.Cu) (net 1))
 (segment (start 149.86 116.84) (end 151.257 118.237) (width 0.3048) (layer F.Cu) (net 1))
 (segment (start 149.9385 111.252) (end 149.9385 108.6665) (width 0.3048) (layer F.Cu) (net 1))
 (segment (start 151.13 109.394741) (end 151.13 107.696) (width 0.1524) (layer F.Cu) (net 2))
 (segment (start 150.876 109.648741) (end 151.13 109.394741) (width 0.1524) (layer F.Cu) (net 2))
 (segment (start 149.86 113.284) (end 150.876 112.268) (width 0.1524) (layer F.Cu) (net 2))
 (segment (start 150.749 107.315) (end 150.02 107.315) (width 0.1524) (layer F.Cu) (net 2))
 (segment (start 151.13 107.696) (end 150.749 107.315) (width 0.1524) (layer F.Cu) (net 2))
 (segment (start 149.86 114.3) (end 149.86 113.284) (width 0.1524) (layer F.Cu) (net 2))
 (segment (start 150.876 112.268) (end 150.876 109.648741) (width 0.1524) (layer F.Cu) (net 2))
 (segment (start 153.478601 108.501201) (end 151.0224 106.045) (width 0.1524) (layer F.Cu) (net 3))
 (segment (start 151.0224 106.045) (end 150.02 106.045) (width 0.1524) (layer F.Cu) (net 3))
 (segment (start 152.4 116.84) (end 153.478601 115.761399) (width 0.1524) (layer F.Cu) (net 3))
 (segment (start 153.478601 115.761399) (end 153.478601 108.501201) (width 0.1524) (layer F.Cu) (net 3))
 (segment (start 153.797 109.8356) (end 156.3176 107.315) (width 0.1524) (layer F.Cu) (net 5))
 (segment (start 156.3176 107.315) (end 157.32 107.315) (width 0.1524) (layer F.Cu) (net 5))
 (segment (start 154.559 112.903) (end 153.797 112.141) (width 0.1524) (layer F.Cu) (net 5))
 (segment (start 155.575 112.903) (end 154.559 112.903) (width 0.1524) (layer F.Cu) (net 5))
 (segment (start 156.21 113.538) (end 155.575 112.903) (width 0.1524) (layer F.Cu) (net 5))
 (segment (start 156.21 115.57) (end 156.21 113.538) (width 0.1524) (layer F.Cu) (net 5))
 (segment (start 157.48 116.84) (end 156.21 115.57) (width 0.1524) (layer F.Cu) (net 5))
 (segment (start 153.797 112.141) (end 153.797 109.8356) (width 0.1524) (layer F.Cu) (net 5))
 (segment (start 157.32 109.0624) (end 157.32 108.585) (width 0.1524) (layer F.Cu) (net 6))
 (segment (start 156.464 109.9184) (end 157.32 109.0624) (width 0.1524) (layer F.Cu) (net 6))
 (segment (start 157.48 113.284) (end 156.464 112.268) (width 0.1524) (layer F.Cu) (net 6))
 (segment (start 157.48 114.3) (end 157.48 113.284) (width 0.1524) (layer F.Cu) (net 6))
 (segment (start 156.464 112.268) (end 156.464 109.9184) (width 0.1524) (layer F.Cu) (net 6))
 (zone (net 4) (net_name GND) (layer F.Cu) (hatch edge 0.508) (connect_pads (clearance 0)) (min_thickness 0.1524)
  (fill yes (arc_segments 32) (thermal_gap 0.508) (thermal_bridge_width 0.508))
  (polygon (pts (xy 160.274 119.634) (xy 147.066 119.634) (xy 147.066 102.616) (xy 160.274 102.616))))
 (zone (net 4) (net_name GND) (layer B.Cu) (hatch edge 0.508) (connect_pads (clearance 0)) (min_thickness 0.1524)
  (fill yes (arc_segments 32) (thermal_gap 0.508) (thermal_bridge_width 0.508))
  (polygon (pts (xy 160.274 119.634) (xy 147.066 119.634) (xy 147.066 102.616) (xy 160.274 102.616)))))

